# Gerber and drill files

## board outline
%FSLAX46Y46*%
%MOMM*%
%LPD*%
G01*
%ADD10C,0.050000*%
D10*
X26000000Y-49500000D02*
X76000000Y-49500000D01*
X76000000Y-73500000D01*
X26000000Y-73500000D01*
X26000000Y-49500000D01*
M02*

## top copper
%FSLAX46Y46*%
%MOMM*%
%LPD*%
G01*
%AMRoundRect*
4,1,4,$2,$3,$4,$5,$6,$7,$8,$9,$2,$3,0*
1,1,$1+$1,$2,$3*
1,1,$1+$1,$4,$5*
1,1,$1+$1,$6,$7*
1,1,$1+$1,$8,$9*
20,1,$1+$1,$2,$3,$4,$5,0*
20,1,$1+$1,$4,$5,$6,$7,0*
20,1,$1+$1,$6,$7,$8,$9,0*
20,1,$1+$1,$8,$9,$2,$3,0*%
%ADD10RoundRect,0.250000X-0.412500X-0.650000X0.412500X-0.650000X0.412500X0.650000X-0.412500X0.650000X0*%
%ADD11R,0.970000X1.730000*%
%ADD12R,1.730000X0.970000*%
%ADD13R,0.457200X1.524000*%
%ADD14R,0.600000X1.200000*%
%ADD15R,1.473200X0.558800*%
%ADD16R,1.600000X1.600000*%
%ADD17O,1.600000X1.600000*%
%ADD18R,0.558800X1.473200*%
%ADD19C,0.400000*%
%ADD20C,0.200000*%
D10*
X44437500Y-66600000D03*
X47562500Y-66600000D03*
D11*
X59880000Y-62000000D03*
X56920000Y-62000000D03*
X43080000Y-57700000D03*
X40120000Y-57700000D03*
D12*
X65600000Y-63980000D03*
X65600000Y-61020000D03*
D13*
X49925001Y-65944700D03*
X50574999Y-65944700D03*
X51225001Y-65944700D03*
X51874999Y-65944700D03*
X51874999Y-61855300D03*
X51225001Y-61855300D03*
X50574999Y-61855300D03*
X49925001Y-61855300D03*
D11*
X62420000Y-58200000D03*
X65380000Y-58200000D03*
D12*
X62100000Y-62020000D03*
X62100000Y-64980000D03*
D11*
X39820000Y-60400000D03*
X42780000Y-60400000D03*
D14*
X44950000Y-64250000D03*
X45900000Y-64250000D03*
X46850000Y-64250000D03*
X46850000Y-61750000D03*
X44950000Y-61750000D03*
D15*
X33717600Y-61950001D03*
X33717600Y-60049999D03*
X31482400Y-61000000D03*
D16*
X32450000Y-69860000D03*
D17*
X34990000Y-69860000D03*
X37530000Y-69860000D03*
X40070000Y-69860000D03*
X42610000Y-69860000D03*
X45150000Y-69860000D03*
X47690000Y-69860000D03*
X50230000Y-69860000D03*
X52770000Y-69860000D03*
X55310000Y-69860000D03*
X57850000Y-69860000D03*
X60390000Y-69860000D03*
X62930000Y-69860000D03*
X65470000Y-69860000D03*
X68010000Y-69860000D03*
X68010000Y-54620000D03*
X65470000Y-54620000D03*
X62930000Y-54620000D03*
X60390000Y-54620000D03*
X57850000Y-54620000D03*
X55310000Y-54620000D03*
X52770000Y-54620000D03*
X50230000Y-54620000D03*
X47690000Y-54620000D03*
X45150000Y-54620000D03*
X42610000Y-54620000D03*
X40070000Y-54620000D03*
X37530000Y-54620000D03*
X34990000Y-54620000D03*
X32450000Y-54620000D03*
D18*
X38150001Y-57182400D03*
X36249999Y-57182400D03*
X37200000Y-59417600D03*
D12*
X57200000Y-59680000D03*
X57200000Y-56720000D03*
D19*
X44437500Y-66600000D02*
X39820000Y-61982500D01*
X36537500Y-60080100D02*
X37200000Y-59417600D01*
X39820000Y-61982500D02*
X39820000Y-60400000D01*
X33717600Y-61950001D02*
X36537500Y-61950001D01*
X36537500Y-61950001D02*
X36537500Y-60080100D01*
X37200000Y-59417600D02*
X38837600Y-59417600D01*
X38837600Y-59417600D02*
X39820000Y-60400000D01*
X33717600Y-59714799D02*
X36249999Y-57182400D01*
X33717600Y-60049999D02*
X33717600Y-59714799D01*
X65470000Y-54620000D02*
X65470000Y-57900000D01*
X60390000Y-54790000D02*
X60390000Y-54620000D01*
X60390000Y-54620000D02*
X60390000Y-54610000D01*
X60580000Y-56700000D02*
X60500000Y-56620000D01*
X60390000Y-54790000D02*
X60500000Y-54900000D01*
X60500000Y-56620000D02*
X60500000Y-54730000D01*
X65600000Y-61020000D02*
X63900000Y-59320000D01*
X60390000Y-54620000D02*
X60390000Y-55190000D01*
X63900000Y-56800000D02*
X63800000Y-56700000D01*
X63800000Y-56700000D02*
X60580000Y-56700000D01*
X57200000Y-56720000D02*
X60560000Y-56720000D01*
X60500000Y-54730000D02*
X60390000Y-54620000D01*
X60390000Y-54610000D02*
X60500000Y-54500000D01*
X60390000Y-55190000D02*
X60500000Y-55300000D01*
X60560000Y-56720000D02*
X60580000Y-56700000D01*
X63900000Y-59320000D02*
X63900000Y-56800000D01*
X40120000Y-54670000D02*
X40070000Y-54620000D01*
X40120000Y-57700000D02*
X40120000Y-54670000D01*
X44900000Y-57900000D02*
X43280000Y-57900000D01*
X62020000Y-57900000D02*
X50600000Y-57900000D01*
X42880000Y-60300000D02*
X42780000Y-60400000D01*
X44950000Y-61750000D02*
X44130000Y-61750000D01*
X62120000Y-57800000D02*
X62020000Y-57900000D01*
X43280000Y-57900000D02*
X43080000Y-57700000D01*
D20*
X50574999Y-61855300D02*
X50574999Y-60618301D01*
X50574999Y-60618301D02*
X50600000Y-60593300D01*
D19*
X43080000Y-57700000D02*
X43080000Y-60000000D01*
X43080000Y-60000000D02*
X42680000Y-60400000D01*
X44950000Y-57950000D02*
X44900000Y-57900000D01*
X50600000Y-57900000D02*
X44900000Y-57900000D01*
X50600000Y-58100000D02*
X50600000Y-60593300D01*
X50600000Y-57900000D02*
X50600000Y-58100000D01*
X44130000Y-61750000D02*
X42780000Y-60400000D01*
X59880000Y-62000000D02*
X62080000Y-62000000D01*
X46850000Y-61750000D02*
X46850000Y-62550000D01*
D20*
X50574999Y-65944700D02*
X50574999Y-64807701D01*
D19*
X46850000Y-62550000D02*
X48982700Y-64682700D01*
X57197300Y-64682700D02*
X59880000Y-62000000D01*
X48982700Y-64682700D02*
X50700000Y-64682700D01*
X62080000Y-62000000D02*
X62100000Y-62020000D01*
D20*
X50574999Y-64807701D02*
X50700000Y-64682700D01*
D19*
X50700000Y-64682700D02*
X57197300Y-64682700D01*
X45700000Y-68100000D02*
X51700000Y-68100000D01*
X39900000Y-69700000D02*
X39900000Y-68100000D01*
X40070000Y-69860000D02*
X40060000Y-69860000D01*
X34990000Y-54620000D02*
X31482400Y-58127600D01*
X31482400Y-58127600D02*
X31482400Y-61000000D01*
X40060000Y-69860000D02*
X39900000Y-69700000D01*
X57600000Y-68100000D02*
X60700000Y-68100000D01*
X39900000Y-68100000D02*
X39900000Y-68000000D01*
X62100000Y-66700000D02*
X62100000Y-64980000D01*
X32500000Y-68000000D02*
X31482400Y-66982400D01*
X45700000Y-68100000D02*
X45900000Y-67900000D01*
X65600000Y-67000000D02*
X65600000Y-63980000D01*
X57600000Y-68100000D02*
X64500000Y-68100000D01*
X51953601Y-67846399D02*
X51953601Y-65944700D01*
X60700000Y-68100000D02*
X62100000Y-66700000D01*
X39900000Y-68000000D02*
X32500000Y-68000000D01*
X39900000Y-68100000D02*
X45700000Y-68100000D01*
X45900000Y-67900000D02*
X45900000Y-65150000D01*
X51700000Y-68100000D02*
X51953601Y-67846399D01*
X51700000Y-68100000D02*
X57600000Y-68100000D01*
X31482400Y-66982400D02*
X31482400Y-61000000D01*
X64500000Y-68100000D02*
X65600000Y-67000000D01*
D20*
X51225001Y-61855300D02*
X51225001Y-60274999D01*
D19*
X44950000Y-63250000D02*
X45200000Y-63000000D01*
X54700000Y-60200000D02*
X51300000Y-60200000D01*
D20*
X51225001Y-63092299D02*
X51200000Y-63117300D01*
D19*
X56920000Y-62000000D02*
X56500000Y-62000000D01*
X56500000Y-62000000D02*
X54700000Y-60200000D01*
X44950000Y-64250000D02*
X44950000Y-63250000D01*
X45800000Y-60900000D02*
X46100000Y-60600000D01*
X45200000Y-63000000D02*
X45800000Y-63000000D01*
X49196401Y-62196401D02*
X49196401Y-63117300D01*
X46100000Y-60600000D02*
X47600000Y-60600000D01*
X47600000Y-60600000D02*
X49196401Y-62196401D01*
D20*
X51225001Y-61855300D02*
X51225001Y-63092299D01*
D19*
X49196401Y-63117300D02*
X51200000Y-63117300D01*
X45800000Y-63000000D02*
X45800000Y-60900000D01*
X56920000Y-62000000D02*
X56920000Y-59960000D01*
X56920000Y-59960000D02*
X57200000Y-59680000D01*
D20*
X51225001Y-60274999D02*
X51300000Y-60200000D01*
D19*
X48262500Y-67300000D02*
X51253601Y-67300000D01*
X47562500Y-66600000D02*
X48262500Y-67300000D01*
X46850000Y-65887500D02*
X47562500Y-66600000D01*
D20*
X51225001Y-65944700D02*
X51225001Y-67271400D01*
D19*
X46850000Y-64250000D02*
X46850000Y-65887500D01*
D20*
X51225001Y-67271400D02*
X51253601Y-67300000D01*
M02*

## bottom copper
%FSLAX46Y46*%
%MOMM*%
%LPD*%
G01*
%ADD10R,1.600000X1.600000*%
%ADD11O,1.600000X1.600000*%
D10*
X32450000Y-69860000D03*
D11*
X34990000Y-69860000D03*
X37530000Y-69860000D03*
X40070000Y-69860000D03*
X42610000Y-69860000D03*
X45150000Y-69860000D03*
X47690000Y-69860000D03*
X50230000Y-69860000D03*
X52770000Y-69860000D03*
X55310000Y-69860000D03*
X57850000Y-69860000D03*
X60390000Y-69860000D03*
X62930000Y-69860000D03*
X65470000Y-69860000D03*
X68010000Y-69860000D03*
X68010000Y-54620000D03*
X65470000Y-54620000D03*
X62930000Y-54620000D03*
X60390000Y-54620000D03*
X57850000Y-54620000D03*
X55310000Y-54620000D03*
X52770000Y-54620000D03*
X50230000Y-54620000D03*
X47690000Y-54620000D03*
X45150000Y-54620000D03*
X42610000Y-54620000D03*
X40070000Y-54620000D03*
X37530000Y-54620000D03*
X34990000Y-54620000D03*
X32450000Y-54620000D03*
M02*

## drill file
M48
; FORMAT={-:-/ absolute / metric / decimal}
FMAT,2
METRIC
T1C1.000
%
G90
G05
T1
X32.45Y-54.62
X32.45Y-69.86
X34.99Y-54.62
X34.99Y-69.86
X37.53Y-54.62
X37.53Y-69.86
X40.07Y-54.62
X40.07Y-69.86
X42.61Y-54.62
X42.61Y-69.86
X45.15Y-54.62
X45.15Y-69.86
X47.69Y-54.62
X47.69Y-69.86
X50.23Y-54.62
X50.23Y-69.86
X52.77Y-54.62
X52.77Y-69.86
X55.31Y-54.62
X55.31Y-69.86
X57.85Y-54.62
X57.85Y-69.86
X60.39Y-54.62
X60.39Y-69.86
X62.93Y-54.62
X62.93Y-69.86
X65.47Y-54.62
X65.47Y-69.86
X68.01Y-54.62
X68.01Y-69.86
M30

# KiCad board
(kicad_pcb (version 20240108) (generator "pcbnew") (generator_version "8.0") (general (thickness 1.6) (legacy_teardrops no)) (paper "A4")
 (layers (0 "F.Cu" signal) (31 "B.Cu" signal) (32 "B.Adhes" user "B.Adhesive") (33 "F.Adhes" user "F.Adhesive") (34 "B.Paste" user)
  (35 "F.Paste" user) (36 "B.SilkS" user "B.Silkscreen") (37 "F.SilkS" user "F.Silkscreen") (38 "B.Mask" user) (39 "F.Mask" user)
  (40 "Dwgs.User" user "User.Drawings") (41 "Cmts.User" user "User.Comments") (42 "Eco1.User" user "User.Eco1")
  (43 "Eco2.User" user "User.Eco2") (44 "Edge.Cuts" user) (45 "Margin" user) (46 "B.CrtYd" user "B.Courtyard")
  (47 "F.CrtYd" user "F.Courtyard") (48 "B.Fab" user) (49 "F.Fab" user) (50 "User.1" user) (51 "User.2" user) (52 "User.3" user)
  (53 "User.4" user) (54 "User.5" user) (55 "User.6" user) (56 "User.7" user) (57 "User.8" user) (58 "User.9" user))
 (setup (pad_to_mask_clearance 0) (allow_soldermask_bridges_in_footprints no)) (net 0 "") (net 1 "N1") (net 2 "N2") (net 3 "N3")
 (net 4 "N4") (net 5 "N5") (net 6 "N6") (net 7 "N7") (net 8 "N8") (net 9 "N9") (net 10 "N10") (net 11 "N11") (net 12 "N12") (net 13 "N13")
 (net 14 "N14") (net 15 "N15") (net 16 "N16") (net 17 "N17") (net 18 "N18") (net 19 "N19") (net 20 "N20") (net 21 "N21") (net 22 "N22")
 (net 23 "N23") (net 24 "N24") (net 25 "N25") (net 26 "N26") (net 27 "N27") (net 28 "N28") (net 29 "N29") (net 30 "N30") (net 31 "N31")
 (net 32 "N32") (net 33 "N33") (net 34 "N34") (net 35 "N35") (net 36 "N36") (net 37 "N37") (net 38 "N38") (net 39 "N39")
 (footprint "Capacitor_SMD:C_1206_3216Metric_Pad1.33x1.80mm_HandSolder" (layer "F.Cu") (at 46 66.6)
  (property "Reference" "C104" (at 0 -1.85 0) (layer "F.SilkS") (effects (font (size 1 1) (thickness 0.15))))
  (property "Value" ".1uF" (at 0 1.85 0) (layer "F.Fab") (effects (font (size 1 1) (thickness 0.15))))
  (pad "1" smd roundrect (at -1.5625 0) (size 1.325 1.8) (layers "F.Cu" "F.Paste" "F.Mask") (roundrect_rratio 0.188679) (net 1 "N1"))
  (pad "2" smd roundrect (at 1.5625 0) (size 1.325 1.8) (layers "F.Cu" "F.Paste" "F.Mask") (roundrect_rratio 0.188679) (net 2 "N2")))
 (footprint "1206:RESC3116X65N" (layer "F.Cu") (at 58.4 62 180)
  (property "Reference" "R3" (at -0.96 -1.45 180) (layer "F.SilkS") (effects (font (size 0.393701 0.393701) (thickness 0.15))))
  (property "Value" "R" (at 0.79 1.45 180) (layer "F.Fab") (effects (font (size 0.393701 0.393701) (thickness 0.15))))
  (pad "1" smd rect (at -1.48 0 180) (size 0.97 1.73) (layers "F.Cu" "F.Paste" "F.Mask") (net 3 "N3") (solder_mask_margin 0.102))
  (pad "2" smd rect (at 1.48 0 180) (size 0.97 1.73) (layers "F.Cu" "F.Paste" "F.Mask") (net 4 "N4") (solder_mask_margin 0.102)))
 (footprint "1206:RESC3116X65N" (layer "F.Cu") (at 41.6 57.7 180)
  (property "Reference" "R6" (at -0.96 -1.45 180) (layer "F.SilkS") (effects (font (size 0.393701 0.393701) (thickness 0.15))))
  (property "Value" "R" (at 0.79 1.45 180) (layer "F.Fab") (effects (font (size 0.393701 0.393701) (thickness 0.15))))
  (pad "1" smd rect (at -1.48 0 180) (size 0.97 1.73) (layers "F.Cu" "F.Paste" "F.Mask") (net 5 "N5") (solder_mask_margin 0.102))
  (pad "2" smd rect (at 1.48 0 180) (size 0.97 1.73) (layers "F.Cu" "F.Paste" "F.Mask") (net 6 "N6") (solder_mask_margin 0.102)))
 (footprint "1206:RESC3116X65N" (layer "F.Cu") (at 65.6 62.5 90)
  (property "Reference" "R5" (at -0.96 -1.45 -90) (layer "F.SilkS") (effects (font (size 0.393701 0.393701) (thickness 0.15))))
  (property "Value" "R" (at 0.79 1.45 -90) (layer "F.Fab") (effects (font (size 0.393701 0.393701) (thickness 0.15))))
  (pad "1" smd rect (at -1.48 0 90) (size 0.97 1.73) (layers "F.Cu" "F.Paste" "F.Mask") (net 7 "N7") (solder_mask_margin 0.102))
  (pad "2" smd rect (at 1.48 0 90) (size 0.97 1.73) (layers "F.Cu" "F.Paste" "F.Mask") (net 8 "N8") (solder_mask_margin 0.102)))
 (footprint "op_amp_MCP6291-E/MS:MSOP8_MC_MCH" (layer "F.Cu") (at 50.9 63.9 90)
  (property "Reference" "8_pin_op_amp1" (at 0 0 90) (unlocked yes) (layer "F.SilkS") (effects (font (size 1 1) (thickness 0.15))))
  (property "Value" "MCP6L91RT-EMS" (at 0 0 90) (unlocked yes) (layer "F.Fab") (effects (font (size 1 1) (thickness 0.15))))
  (pad "1" smd rect (at -2.0447 -0.974999 90) (size 1.524 0.4572) (layers "F.Cu" "F.Paste" "F.Mask") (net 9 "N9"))
  (pad "2" smd rect (at -2.0447 -0.325001 90) (size 1.524 0.4572) (layers "F.Cu" "F.Paste" "F.Mask") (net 3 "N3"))
  (pad "3" smd rect (at -2.0447 0.325001 90) (size 1.524 0.4572) (layers "F.Cu" "F.Paste" "F.Mask") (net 2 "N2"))
  (pad "4" smd rect (at -2.0447 0.974999 90) (size 1.524 0.4572) (layers "F.Cu" "F.Paste" "F.Mask") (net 7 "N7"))
  (pad "5" smd rect (at 2.0447 0.974999 90) (size 1.524 0.4572) (layers "F.Cu" "F.Paste" "F.Mask") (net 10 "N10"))
  (pad "6" smd rect (at 2.0447 0.325001 90) (size 1.524 0.4572) (layers "F.Cu" "F.Paste" "F.Mask") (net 4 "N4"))
  (pad "7" smd rect (at 2.0447 -0.325001 90) (size 1.524 0.4572) (layers "F.Cu" "F.Paste" "F.Mask") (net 5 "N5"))
  (pad "8" smd rect (at 2.0447 -0.974999 90) (size 1.524 0.4572) (layers "F.Cu" "F.Paste" "F.Mask") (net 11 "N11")))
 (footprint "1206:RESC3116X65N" (layer "F.Cu") (at 63.9 58.2)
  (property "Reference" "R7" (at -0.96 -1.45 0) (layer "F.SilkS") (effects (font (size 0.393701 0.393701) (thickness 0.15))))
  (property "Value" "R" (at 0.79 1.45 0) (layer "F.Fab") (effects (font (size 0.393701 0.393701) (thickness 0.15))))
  (pad "1" smd rect (at -1.48 0) (size 0.97 1.73) (layers "F.Cu" "F.Paste" "F.Mask") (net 5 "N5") (solder_mask_margin 0.102))
  (pad "2" smd rect (at 1.48 0) (size 0.97 1.73) (layers "F.Cu" "F.Paste" "F.Mask") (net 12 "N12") (solder_mask_margin 0.102)))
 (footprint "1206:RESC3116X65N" (layer "F.Cu") (at 62.1 63.5 -90)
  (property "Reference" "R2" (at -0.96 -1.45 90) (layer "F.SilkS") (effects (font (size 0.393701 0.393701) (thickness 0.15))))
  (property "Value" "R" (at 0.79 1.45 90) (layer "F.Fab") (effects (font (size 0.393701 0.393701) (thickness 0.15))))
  (pad "1" smd rect (at -1.48 0 270) (size 0.97 1.73) (layers "F.Cu" "F.Paste" "F.Mask") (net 3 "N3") (solder_mask_margin 0.102))
  (pad "2" smd rect (at 1.48 0 270) (size 0.97 1.73) (layers "F.Cu" "F.Paste" "F.Mask") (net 7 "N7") (solder_mask_margin 0.102)))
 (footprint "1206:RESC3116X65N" (layer "F.Cu") (at 41.3 60.4)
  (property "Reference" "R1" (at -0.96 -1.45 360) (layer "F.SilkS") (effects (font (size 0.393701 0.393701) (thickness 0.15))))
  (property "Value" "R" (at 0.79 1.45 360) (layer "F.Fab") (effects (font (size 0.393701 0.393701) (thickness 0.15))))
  (pad "1" smd rect (at -1.48 0) (size 0.97 1.73) (layers "F.Cu" "F.Paste" "F.Mask") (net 1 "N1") (solder_mask_margin 0.102))
  (pad "2" smd rect (at 1.48 0) (size 0.97 1.73) (layers "F.Cu" "F.Paste" "F.Mask") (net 5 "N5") (solder_mask_margin 0.102)))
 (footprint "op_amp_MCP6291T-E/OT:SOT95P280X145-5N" (layer "F.Cu") (at 45.9 63 90)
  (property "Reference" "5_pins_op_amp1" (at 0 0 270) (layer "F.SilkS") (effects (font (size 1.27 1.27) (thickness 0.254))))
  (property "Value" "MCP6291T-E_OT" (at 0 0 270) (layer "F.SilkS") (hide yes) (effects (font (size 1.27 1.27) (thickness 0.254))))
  (pad "1" smd rect (at -1.25 -0.95 180) (size 0.6 1.2) (layers "F.Cu" "F.Paste" "F.Mask") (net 4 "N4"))
  (pad "2" smd rect (at -1.25 0 180) (size 0.6 1.2) (layers "F.Cu" "F.Paste" "F.Mask") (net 7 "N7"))
  (pad "3" smd rect (at -1.25 0.95 180) (size 0.6 1.2) (layers "F.Cu" "F.Paste" "F.Mask") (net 2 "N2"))
  (pad "4" smd rect (at 1.25 0.95 180) (size 0.6 1.2) (layers "F.Cu" "F.Paste" "F.Mask") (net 3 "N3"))
  (pad "5" smd rect (at 1.25 -0.95 180) (size 0.6 1.2) (layers "F.Cu" "F.Paste" "F.Mask") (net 5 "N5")))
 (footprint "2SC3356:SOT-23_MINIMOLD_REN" (layer "F.Cu") (at 32.6 61 90)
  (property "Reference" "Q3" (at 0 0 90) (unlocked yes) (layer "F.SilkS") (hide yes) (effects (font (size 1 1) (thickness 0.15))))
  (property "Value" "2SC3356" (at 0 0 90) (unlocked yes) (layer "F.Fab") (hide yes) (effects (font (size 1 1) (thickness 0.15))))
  (pad "1" smd rect (at -0.950001 1.1176 90) (size 0.5588 1.4732) (layers "F.Cu" "F.Paste" "F.Mask") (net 1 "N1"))
  (pad "2" smd rect (at 0.950001 1.1176 90) (size 0.5588 1.4732) (layers "F.Cu" "F.Paste" "F.Mask") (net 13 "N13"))
  (pad "3" smd rect (at 0 -1.1176 90) (size 0.5588 1.4732) (layers "F.Cu" "F.Paste" "F.Mask") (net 7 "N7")))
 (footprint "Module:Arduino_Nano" (layer "F.Cu") (at 32.45 69.86 90)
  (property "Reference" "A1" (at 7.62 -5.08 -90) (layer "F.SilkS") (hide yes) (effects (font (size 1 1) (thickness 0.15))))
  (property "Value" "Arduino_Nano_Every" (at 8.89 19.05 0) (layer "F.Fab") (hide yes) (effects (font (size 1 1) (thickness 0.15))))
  (pad "1" thru_hole rect (at 0 0 90) (size 1.6 1.6) (drill 1) (layers "*.Cu" "*.Mask") (remove_unused_layers no) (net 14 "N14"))
  (pad "2" thru_hole oval (at 0 2.54 90) (size 1.6 1.6) (drill 1) (layers "*.Cu" "*.Mask") (remove_unused_layers no) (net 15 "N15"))
  (pad "3" thru_hole oval (at 0 5.08 90) (size 1.6 1.6) (drill 1) (layers "*.Cu" "*.Mask") (remove_unused_layers no) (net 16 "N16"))
  (pad "4" thru_hole oval (at 0 7.62 90) (size 1.6 1.6) (drill 1) (layers "*.Cu" "*.Mask") (remove_unused_layers no) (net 7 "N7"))
  (pad "5" thru_hole oval (at 0 10.16 90) (size 1.6 1.6) (drill 1) (layers "*.Cu" "*.Mask") (remove_unused_layers no) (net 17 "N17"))
  (pad "6" thru_hole oval (at 0 12.7 90) (size 1.6 1.6) (drill 1) (layers "*.Cu" "*.Mask") (remove_unused_layers no) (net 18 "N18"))
  (pad "7" thru_hole oval (at 0 15.24 90) (size 1.6 1.6) (drill 1) (layers "*.Cu" "*.Mask") (remove_unused_layers no) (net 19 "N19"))
  (pad "8" thru_hole oval (at 0 17.78 90) (size 1.6 1.6) (drill 1) (layers "*.Cu" "*.Mask") (remove_unused_layers no) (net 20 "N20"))
  (pad "9" thru_hole oval (at 0 20.32 90) (size 1.6 1.6) (drill 1) (layers "*.Cu" "*.Mask") (remove_unused_layers no) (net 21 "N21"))
  (pad "10" thru_hole oval (at 0 22.86 90) (size 1.6 1.6) (drill 1) (layers "*.Cu" "*.Mask") (remove_unused_layers no) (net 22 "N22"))
  (pad "11" thru_hole oval (at 0 25.4 90) (size 1.6 1.6) (drill 1) (layers "*.Cu" "*.Mask") (remove_unused_layers no) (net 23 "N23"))
  (pad "12" thru_hole oval (at 0 27.94 90) (size 1.6 1.6) (drill 1) (layers "*.Cu" "*.Mask") (remove_unused_layers no) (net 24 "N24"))
  (pad "13" thru_hole oval (at 0 30.48 90) (size 1.6 1.6) (drill 1) (layers "*.Cu" "*.Mask") (remove_unused_layers no) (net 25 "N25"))
  (pad "14" thru_hole oval (at 0 33.02 90) (size 1.6 1.6) (drill 1) (layers "*.Cu" "*.Mask") (remove_unused_layers no) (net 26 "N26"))
  (pad "15" thru_hole oval (at 0 35.56 90) (size 1.6 1.6) (drill 1) (layers "*.Cu" "*.Mask") (remove_unused_layers no) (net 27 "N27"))
  (pad "16" thru_hole oval (at 15.24 35.56 90) (size 1.6 1.6) (drill 1) (layers "*.Cu" "*.Mask") (remove_unused_layers no) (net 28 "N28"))
  (pad "17" thru_hole oval (at 15.24 33.02 90) (size 1.6 1.6) (drill 1) (layers "*.Cu" "*.Mask") (remove_unused_layers no) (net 12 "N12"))
  (pad "18" thru_hole oval (at 15.24 30.48 90) (size 1.6 1.6) (drill 1) (layers "*.Cu" "*.Mask") (remove_unused_layers no) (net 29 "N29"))
  (pad "19" thru_hole oval (at 15.24 27.94 90) (size 1.6 1.6) (drill 1) (layers "*.Cu" "*.Mask") (remove_unused_layers no) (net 8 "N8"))
  (pad "20" thru_hole oval (at 15.24 25.4 90) (size 1.6 1.6) (drill 1) (layers "*.Cu" "*.Mask") (remove_unused_layers no) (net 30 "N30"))
  (pad "21" thru_hole oval (at 15.24 22.86 90) (size 1.6 1.6) (drill 1) (layers "*.Cu" "*.Mask") (remove_unused_layers no) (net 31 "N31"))
  (pad "22" thru_hole oval (at 15.24 20.32 90) (size 1.6 1.6) (drill 1) (layers "*.Cu" "*.Mask") (remove_unused_layers no) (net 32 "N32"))
  (pad "23" thru_hole oval (at 15.24 17.78 90) (size 1.6 1.6) (drill 1) (layers "*.Cu" "*.Mask") (remove_unused_layers no) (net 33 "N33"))
  (pad "24" thru_hole oval (at 15.24 15.24 90) (size 1.6 1.6) (drill 1) (layers "*.Cu" "*.Mask") (remove_unused_layers no) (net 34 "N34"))
  (pad "25" thru_hole oval (at 15.24 12.7 90) (size 1.6 1.6) (drill 1) (layers "*.Cu" "*.Mask") (remove_unused_layers no) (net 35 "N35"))
  (pad "26" thru_hole oval (at 15.24 10.16 90) (size 1.6 1.6) (drill 1) (layers "*.Cu" "*.Mask") (remove_unused_layers no) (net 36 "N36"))
  (pad "27" thru_hole oval (at 15.24 7.62 90) (size 1.6 1.6) (drill 1) (layers "*.Cu" "*.Mask") (remove_unused_layers no) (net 6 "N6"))
  (pad "28" thru_hole oval (at 15.24 5.08 90) (size 1.6 1.6) (drill 1) (layers "*.Cu" "*.Mask") (remove_unused_layers no) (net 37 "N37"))
  (pad "29" thru_hole oval (at 15.24 2.54 90) (size 1.6 1.6) (drill 1) (layers "*.Cu" "*.Mask") (remove_unused_layers no) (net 7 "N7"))
  (pad "30" thru_hole oval (at 15.24 0 90) (size 1.6 1.6) (drill 1) (layers "*.Cu" "*.Mask") (remove_unused_layers no) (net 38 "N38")))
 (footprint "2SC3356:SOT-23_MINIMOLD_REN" (layer "F.Cu") (at 37.2 58.3 180)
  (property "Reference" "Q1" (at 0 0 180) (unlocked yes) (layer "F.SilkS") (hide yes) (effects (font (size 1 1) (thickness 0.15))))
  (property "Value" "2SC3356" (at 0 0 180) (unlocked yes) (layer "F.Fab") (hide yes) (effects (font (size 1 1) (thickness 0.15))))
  (pad "1" smd rect (at -0.950001 1.1176 180) (size 0.5588 1.4732) (layers "F.Cu" "F.Paste" "F.Mask") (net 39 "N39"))
  (pad "2" smd rect (at 0.950001 1.1176 180) (size 0.5588 1.4732) (layers "F.Cu" "F.Paste" "F.Mask") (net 13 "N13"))
  (pad "3" smd rect (at 0 -1.1176 180) (size 0.5588 1.4732) (layers "F.Cu" "F.Paste" "F.Mask") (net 1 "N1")))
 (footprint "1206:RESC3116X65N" (layer "F.Cu") (at 57.2 58.2 90)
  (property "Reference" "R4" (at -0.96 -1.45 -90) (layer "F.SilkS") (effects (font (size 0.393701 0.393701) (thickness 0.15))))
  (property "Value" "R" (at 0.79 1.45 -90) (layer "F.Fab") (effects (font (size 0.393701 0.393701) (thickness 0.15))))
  (pad "1" smd rect (at -1.48 0 90) (size 0.97 1.73) (layers "F.Cu" "F.Paste" "F.Mask") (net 4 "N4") (solder_mask_margin 0.102))
  (pad "2" smd rect (at 1.48 0 90) (size 0.97 1.73) (layers "F.Cu" "F.Paste" "F.Mask") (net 8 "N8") (solder_mask_margin 0.102)))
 (gr_rect (start 26 49.5) (end 76 73.5) (stroke (width 0.05) (type default)) (fill none) (layer "Edge.Cuts"))
 (segment (start 44.4375 66.6) (end 39.82 61.9825) (width 0.4) (layer "F.Cu") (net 1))
 (segment (start 36.5375 60.0801) (end 37.2 59.4176) (width 0.4) (layer "F.Cu") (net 1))
 (segment (start 39.82 61.9825) (end 39.82 60.4) (width 0.4) (layer "F.Cu") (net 1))
 (segment (start 33.7176 61.950001) (end 36.5375 61.950001) (width 0.4) (layer "F.Cu") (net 1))
 (segment (start 36.5375 61.950001) (end 36.5375 60.0801) (width 0.4) (layer "F.Cu") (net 1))
 (segment (start 37.2 59.4176) (end 38.8376 59.4176) (width 0.4) (layer "F.Cu") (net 1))
 (segment (start 38.8376 59.4176) (end 39.82 60.4) (width 0.4) (layer "F.Cu") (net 1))
 (segment (start 33.7176 59.714799) (end 36.249999 57.1824) (width 0.4) (layer "F.Cu") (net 13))
 (segment (start 33.7176 60.049999) (end 33.7176 59.714799) (width 0.4) (layer "F.Cu") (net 13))
 (segment (start 65.47 54.62) (end 65.47 57.9) (width 0.4) (layer "F.Cu") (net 12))
 (segment (start 60.39 54.79) (end 60.39 54.62) (width 0.4) (layer "F.Cu") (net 8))
 (segment (start 60.39 54.62) (end 60.39 54.61) (width 0.4) (layer "F.Cu") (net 8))
 (segment (start 60.58 56.7) (end 60.5 56.62) (width 0.4) (layer "F.Cu") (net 8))
 (segment (start 60.39 54.79) (end 60.5 54.9) (width 0.4) (layer "F.Cu") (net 8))
 (segment (start 60.5 56.62) (end 60.5 54.73) (width 0.4) (layer "F.Cu") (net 8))
 (segment (start 65.6 61.02) (end 63.9 59.32) (width 0.4) (layer "F.Cu") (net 8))
 (segment (start 60.39 54.62) (end 60.39 55.19) (width 0.4) (layer "F.Cu") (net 8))
 (segment (start 63.9 56.8) (end 63.8 56.7) (width 0.4) (layer "F.Cu") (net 8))
 (segment (start 63.8 56.7) (end 60.58 56.7) (width 0.4) (layer "F.Cu") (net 8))
 (segment (start 57.2 56.72) (end 60.56 56.72) (width 0.4) (layer "F.Cu") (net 8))
 (segment (start 60.5 54.73) (end 60.39 54.62) (width 0.4) (layer "F.Cu") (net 8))
 (segment (start 60.39 54.61) (end 60.5 54.5) (width 0.4) (layer "F.Cu") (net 8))
 (segment (start 60.39 55.19) (end 60.5 55.3) (width 0.4) (layer "F.Cu") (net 8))
 (segment (start 60.56 56.72) (end 60.58 56.7) (width 0.4) (layer "F.Cu") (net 8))
 (segment (start 63.9 59.32) (end 63.9 56.8) (width 0.4) (layer "F.Cu") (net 8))
 (segment (start 40.12 54.67) (end 40.07 54.62) (width 0.4) (layer "F.Cu") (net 6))
 (segment (start 40.12 57.7) (end 40.12 54.67) (width 0.4) (layer "F.Cu") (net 6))
 (segment (start 44.9 57.9) (end 43.28 57.9) (width 0.4) (layer "F.Cu") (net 5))
 (segment (start 62.02 57.9) (end 50.6 57.9) (width 0.4) (layer "F.Cu") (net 5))
 (segment (start 42.88 60.3) (end 42.78 60.4) (width 0.4) (layer "F.Cu") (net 5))
 (segment (start 44.95 61.75) (end 44.13 61.75) (width 0.4) (layer "F.Cu") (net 5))
 (segment (start 62.12 57.8) (end 62.02 57.9) (width 0.4) (layer "F.Cu") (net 5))
 (segment (start 43.28 57.9) (end 43.08 57.7) (width 0.4) (layer "F.Cu") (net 5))
 (segment (start 50.574999 61.8553) (end 50.574999 60.618301) (width 0.2) (layer "F.Cu") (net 5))
 (segment (start 50.574999 60.618301) (end 50.6 60.5933) (width 0.2) (layer "F.Cu") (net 5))
 (segment (start 43.08 57.7) (end 43.08 60) (width 0.4) (layer "F.Cu") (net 5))
 (segment (start 43.08 60) (end 42.68 60.4) (width 0.4) (layer "F.Cu") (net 5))
 (segment (start 44.95 57.95) (end 44.9 57.9) (width 0.4) (layer "F.Cu") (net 5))
 (segment (start 50.6 57.9) (end 44.9 57.9) (width 0.4) (layer "F.Cu") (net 5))
 (segment (start 50.6 58.1) (end 50.6 60.5933) (width 0.4) (layer "F.Cu") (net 5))
 (segment (start 50.6 57.9) (end 50.6 58.1) (width 0.4) (layer "F.Cu") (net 5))
 (segment (start 44.13 61.75) (end 42.78 60.4) (width 0.4) (layer "F.Cu") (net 5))
 (segment (start 59.88 62) (end 62.08 62) (width 0.4) (layer "F.Cu") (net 3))
 (segment (start 46.85 61.75) (end 46.85 62.55) (width 0.4) (layer "F.Cu") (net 3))
 (segment (start 50.574999 65.9447) (end 50.574999 64.807701) (width 0.2) (layer "F.Cu") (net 3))
 (segment (start 46.85 62.55) (end 48.9827 64.6827) (width 0.4) (layer "F.Cu") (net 3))
 (segment (start 57.1973 64.6827) (end 59.88 62) (width 0.4) (layer "F.Cu") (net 3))
 (segment (start 48.9827 64.6827) (end 50.7 64.6827) (width 0.4) (layer "F.Cu") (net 3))
 (segment (start 62.08 62) (end 62.1 62.02) (width 0.4) (layer "F.Cu") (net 3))
 (segment (start 50.574999 64.807701) (end 50.7 64.6827) (width 0.2) (layer "F.Cu") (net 3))
 (segment (start 50.7 64.6827) (end 57.1973 64.6827) (width 0.4) (layer "F.Cu") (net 3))
 (segment (start 45.7 68.1) (end 51.7 68.1) (width 0.4) (layer "F.Cu") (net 7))
 (segment (start 39.9 69.7) (end 39.9 68.1) (width 0.4) (layer "F.Cu") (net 7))
 (segment (start 40.07 69.86) (end 40.06 69.86) (width 0.4) (layer "F.Cu") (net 7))
 (segment (start 34.99 54.62) (end 31.4824 58.1276) (width 0.4) (layer "F.Cu") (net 7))
 (segment (start 31.4824 58.1276) (end 31.4824 61) (width 0.4) (layer "F.Cu") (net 7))
 (segment (start 40.06 69.86) (end 39.9 69.7) (width 0.4) (layer "F.Cu") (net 7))
 (segment (start 57.6 68.1) (end 60.7 68.1) (width 0.4) (layer "F.Cu") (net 7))
 (segment (start 39.9 68.1) (end 39.9 68) (width 0.4) (layer "F.Cu") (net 7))
 (segment (start 62.1 66.7) (end 62.1 64.98) (width 0.4) (layer "F.Cu") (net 7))
 (segment (start 32.5 68) (end 31.4824 66.9824) (width 0.4) (layer "F.Cu") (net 7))
 (segment (start 45.7 68.1) (end 45.9 67.9) (width 0.4) (layer "F.Cu") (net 7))
 (segment (start 65.6 67) (end 65.6 63.98) (width 0.4) (layer "F.Cu") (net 7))
 (segment (start 57.6 68.1) (end 64.5 68.1) (width 0.4) (layer "F.Cu") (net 7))
 (segment (start 51.953601 67.846399) (end 51.953601 65.9447) (width 0.4) (layer "F.Cu") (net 7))
 (segment (start 60.7 68.1) (end 62.1 66.7) (width 0.4) (layer "F.Cu") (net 7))
 (segment (start 39.9 68) (end 32.5 68) (width 0.4) (layer "F.Cu") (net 7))
 (segment (start 39.9 68.1) (end 45.7 68.1) (width 0.4) (layer "F.Cu") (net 7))
 (segment (start 45.9 67.9) (end 45.9 65.15) (width 0.4) (layer "F.Cu") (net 7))
 (segment (start 51.7 68.1) (end 51.953601 67.846399) (width 0.4) (layer "F.Cu") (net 7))
 (segment (start 51.7 68.1) (end 57.6 68.1) (width 0.4) (layer "F.Cu") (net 7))
 (segment (start 31.4824 66.9824) (end 31.4824 61) (width 0.4) (layer "F.Cu") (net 7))
 (segment (start 64.5 68.1) (end 65.6 67) (width 0.4) (layer "F.Cu") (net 7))
 (segment (start 51.225001 61.8553) (end 51.225001 60.274999) (width 0.2) (layer "F.Cu") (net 4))
 (segment (start 44.95 63.25) (end 45.2 63) (width 0.4) (layer "F.Cu") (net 4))
 (segment (start 54.7 60.2) (end 51.3 60.2) (width 0.4) (layer "F.Cu") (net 4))
 (segment (start 51.225001 63.092299) (end 51.2 63.1173) (width 0.2) (layer "F.Cu") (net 4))
 (segment (start 56.92 62) (end 56.5 62) (width 0.4) (layer "F.Cu") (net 4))
 (segment (start 56.5 62) (end 54.7 60.2) (width 0.4) (layer "F.Cu") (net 4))
 (segment (start 44.95 64.25) (end 44.95 63.25) (width 0.4) (layer "F.Cu") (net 4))
 (segment (start 45.8 60.9) (end 46.1 60.6) (width 0.4) (layer "F.Cu") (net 4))
 (segment (start 45.2 63) (end 45.8 63) (width 0.4) (layer "F.Cu") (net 4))
 (segment (start 49.196401 62.196401) (end 49.196401 63.1173) (width 0.4) (layer "F.Cu") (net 4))
 (segment (start 46.1 60.6) (end 47.6 60.6) (width 0.4) (layer "F.Cu") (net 4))
 (segment (start 47.6 60.6) (end 49.196401 62.196401) (width 0.4) (layer "F.Cu") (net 4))
 (segment (start 51.225001 61.8553) (end 51.225001 63.092299) (width 0.2) (layer "F.Cu") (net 4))
 (segment (start 49.196401 63.1173) (end 51.2 63.1173) (width 0.4) (layer "F.Cu") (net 4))
 (segment (start 45.8 63) (end 45.8 60.9) (width 0.4) (layer "F.Cu") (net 4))
 (segment (start 56.92 62) (end 56.92 59.96) (width 0.4) (layer "F.Cu") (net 4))
 (segment (start 56.92 59.96) (end 57.2 59.68) (width 0.4) (layer "F.Cu") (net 4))
 (segment (start 51.225001 60.274999) (end 51.3 60.2) (width 0.2) (layer "F.Cu") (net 4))
 (segment (start 48.2625 67.3) (end 51.253601 67.3) (width 0.4) (layer "F.Cu") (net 2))
 (segment (start 47.5625 66.6) (end 48.2625 67.3) (width 0.4) (layer "F.Cu") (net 2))
 (segment (start 46.85 65.8875) (end 47.5625 66.6) (width 0.4) (layer "F.Cu") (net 2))
 (segment (start 51.225001 65.9447) (end 51.225001 67.2714) (width 0.2) (layer "F.Cu") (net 2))
 (segment (start 46.85 64.25) (end 46.85 65.8875) (width 0.4) (layer "F.Cu") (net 2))
 (segment (start 51.225001 67.2714) (end 51.253601 67.3) (width 0.2) (layer "F.Cu") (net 2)))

